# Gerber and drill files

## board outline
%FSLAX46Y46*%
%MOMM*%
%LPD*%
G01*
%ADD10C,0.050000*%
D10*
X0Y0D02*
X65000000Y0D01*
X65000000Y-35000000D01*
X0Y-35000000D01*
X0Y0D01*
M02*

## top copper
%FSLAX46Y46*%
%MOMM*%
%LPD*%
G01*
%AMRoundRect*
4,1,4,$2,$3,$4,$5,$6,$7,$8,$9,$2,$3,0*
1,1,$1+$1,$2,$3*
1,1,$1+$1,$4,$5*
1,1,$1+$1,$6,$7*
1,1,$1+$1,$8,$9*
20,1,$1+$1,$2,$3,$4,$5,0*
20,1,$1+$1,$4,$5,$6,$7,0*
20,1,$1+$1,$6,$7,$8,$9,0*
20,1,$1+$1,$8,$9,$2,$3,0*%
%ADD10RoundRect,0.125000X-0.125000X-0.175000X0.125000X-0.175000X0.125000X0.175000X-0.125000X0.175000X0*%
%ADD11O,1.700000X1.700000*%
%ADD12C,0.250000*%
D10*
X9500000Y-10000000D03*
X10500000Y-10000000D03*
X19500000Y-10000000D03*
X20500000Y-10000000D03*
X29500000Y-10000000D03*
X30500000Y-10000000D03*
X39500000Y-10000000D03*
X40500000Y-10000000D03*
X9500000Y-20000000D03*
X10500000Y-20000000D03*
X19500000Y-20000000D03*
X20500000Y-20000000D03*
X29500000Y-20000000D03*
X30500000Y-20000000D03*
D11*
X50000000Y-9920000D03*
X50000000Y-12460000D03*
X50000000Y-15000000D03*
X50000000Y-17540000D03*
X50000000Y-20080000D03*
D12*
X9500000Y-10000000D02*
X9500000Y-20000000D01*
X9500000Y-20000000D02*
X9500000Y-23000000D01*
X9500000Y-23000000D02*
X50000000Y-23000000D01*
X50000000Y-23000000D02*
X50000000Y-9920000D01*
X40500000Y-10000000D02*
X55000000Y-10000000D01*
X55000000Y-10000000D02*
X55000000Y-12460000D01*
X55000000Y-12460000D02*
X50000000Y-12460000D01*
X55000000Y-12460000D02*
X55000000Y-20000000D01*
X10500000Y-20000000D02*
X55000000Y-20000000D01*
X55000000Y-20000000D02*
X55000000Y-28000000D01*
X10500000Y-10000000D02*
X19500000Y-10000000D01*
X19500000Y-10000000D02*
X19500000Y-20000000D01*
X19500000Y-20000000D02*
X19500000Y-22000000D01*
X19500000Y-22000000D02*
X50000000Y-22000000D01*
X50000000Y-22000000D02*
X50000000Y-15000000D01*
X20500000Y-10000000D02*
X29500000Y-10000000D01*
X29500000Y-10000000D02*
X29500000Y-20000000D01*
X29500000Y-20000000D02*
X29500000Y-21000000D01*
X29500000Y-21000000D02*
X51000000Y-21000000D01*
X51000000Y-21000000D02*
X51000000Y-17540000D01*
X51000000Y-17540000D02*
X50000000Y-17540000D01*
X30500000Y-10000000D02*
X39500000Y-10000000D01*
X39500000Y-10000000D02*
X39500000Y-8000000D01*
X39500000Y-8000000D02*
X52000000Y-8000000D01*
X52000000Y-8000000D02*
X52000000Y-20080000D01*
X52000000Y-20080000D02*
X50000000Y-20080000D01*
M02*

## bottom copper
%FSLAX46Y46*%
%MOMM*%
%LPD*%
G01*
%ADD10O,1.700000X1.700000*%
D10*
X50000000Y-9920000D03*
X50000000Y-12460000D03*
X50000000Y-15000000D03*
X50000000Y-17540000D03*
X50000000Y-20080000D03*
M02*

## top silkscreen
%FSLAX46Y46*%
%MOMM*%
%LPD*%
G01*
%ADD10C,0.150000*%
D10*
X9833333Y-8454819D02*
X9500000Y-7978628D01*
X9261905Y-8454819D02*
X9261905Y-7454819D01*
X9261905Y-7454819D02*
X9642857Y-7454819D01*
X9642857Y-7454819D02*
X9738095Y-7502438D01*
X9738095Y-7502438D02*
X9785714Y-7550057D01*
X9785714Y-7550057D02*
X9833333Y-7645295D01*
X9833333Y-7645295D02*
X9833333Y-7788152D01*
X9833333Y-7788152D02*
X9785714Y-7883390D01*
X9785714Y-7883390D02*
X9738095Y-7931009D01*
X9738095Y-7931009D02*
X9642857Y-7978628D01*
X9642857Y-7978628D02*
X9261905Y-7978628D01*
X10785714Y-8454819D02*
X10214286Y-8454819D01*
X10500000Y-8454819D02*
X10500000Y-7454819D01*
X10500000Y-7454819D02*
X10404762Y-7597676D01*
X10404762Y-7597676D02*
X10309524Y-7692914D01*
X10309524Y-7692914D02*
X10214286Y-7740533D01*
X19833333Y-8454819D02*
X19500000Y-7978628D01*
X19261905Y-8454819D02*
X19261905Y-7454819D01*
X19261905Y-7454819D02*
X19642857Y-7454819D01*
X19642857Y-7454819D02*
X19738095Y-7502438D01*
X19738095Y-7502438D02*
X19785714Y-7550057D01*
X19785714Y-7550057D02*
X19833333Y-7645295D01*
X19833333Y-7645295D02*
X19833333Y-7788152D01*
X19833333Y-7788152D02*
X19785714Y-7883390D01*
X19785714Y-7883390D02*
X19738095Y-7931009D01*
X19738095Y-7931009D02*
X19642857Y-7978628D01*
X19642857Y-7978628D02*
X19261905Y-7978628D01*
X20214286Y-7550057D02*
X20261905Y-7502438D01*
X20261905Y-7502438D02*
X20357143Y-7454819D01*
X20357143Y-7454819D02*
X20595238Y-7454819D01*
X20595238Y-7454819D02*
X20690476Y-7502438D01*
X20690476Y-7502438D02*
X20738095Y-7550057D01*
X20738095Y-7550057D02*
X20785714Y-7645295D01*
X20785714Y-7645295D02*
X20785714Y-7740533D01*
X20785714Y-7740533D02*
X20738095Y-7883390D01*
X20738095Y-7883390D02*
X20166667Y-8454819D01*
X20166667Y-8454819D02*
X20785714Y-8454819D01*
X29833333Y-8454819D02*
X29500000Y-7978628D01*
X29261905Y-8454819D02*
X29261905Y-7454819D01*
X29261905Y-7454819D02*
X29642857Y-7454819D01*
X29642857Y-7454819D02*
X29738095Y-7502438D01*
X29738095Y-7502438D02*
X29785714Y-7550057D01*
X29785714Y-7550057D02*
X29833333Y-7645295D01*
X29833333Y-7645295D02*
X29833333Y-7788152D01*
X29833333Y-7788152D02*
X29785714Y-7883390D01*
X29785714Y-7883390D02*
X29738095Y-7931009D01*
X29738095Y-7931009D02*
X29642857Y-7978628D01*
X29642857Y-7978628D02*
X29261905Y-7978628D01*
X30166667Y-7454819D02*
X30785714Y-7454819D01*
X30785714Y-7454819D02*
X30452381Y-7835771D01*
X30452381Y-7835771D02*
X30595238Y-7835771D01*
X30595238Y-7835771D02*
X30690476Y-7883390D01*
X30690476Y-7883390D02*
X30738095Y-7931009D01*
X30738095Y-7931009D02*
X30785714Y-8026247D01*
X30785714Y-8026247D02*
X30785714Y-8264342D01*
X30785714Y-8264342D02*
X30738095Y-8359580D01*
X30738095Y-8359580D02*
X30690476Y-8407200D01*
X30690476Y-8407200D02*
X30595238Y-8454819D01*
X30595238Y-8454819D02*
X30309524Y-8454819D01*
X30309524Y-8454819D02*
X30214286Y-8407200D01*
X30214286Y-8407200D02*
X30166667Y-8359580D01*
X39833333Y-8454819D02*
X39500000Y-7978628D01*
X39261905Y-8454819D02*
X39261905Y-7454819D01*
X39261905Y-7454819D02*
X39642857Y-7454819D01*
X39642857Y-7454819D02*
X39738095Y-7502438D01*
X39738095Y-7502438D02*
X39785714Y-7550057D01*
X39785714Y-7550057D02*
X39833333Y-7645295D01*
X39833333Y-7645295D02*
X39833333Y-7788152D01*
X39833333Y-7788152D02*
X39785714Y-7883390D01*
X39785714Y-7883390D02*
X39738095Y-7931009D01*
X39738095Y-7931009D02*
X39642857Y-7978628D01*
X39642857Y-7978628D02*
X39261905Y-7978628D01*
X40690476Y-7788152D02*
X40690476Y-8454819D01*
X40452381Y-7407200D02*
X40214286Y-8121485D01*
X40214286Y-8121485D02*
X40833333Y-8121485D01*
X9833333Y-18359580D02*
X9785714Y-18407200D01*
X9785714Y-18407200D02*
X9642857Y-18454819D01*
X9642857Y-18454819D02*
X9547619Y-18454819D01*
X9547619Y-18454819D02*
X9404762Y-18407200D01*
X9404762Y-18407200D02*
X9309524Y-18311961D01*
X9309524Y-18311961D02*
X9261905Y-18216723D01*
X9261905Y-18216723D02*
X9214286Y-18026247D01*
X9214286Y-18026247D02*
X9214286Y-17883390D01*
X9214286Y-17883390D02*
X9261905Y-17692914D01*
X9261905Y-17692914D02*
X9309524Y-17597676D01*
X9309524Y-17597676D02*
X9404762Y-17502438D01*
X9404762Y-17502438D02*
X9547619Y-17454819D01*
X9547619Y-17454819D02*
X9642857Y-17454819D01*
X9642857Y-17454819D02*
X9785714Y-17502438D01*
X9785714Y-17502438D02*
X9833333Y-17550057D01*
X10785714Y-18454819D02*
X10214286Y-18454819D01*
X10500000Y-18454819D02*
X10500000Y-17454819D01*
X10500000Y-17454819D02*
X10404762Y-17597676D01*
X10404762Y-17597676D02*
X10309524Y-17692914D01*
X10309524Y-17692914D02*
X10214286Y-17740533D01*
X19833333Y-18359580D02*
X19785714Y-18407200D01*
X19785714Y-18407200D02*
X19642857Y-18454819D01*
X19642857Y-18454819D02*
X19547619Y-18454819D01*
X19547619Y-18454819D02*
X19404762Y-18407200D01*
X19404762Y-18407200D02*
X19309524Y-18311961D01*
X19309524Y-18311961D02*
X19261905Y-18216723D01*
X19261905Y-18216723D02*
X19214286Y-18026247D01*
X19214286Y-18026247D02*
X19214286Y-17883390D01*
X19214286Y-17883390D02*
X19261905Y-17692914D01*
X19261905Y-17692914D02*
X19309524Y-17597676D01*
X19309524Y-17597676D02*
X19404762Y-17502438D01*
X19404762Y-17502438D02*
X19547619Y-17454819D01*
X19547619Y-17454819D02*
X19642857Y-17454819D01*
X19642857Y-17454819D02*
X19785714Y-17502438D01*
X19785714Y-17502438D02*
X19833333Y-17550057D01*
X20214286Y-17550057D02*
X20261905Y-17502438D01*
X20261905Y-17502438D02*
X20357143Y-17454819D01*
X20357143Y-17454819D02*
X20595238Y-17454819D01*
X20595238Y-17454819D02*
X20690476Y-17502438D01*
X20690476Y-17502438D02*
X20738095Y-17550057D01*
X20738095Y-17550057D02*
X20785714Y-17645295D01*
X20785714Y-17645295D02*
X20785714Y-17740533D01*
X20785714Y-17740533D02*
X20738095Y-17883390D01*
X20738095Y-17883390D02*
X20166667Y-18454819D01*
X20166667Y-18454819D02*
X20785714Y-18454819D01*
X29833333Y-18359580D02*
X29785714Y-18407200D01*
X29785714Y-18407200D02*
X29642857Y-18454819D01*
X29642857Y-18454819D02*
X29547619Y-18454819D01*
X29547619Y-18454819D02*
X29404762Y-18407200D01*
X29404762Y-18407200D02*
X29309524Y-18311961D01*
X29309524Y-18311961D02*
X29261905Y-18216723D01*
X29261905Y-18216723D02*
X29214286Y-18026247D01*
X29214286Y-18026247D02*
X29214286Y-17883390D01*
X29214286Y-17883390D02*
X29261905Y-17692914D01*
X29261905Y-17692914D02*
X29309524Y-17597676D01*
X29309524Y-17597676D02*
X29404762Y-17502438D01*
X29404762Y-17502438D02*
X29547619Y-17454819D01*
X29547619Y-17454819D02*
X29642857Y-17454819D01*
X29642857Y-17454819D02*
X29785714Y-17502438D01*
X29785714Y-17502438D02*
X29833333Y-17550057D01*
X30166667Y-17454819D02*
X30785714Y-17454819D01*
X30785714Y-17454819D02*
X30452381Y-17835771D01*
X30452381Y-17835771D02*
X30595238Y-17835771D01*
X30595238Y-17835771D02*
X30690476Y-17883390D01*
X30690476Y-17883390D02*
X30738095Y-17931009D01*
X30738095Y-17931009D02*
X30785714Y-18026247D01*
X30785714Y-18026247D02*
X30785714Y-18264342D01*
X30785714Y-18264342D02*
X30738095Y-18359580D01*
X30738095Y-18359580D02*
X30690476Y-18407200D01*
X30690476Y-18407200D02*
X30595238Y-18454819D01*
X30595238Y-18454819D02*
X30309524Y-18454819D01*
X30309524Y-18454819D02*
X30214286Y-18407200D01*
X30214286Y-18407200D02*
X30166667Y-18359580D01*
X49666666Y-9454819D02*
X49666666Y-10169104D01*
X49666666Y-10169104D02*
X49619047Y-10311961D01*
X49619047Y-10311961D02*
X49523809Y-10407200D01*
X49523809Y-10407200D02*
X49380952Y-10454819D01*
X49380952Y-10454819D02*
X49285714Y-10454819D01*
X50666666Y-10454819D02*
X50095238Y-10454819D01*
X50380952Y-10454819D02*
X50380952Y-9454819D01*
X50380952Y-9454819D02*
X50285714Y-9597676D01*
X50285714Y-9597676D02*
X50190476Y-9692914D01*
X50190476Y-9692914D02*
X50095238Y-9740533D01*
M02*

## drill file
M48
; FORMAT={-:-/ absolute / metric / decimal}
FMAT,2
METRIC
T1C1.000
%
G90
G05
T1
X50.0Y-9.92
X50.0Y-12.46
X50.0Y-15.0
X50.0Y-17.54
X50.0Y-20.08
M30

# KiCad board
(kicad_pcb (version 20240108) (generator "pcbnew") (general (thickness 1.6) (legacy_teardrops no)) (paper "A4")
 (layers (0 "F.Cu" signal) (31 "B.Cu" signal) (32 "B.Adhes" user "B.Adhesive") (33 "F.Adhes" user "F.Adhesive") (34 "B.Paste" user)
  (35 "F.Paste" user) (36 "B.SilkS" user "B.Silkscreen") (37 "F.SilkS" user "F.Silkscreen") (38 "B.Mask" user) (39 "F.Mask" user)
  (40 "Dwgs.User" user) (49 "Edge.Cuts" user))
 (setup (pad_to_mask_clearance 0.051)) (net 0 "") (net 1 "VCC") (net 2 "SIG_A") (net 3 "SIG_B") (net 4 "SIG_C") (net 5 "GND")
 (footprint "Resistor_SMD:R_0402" (layer "F.Cu") (at 10 10)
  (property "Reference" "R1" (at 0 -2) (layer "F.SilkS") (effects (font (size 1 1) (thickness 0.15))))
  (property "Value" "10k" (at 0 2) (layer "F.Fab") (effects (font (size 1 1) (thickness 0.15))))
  (pad "1" smd roundrect (at -0.5 0) (size 0.5 0.6) (layers "F.Cu" "F.Paste" "F.Mask") (roundrect_rratio 0.25) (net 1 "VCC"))
  (pad "2" smd roundrect (at 0.5 0) (size 0.5 0.6) (layers "F.Cu" "F.Paste" "F.Mask") (roundrect_rratio 0.25) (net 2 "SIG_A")))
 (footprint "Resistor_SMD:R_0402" (layer "F.Cu") (at 20 10)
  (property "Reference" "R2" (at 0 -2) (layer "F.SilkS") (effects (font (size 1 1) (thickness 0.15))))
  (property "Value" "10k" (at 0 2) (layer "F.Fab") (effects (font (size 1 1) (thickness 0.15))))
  (pad "1" smd roundrect (at -0.5 0) (size 0.5 0.6) (layers "F.Cu" "F.Paste" "F.Mask") (roundrect_rratio 0.25) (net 2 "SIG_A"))
  (pad "2" smd roundrect (at 0.5 0) (size 0.5 0.6) (layers "F.Cu" "F.Paste" "F.Mask") (roundrect_rratio 0.25) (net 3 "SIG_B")))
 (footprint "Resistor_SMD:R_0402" (layer "F.Cu") (at 30 10)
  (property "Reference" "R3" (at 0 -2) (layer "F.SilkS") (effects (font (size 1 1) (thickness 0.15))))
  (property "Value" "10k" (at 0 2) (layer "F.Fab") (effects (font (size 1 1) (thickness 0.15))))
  (pad "1" smd roundrect (at -0.5 0) (size 0.5 0.6) (layers "F.Cu" "F.Paste" "F.Mask") (roundrect_rratio 0.25) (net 3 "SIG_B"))
  (pad "2" smd roundrect (at 0.5 0) (size 0.5 0.6) (layers "F.Cu" "F.Paste" "F.Mask") (roundrect_rratio 0.25) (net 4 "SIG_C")))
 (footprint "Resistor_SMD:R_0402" (layer "F.Cu") (at 40 10)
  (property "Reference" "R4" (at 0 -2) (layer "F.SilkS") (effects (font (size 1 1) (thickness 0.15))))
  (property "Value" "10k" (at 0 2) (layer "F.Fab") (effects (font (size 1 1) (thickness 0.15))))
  (pad "1" smd roundrect (at -0.5 0) (size 0.5 0.6) (layers "F.Cu" "F.Paste" "F.Mask") (roundrect_rratio 0.25) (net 4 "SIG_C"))
  (pad "2" smd roundrect (at 0.5 0) (size 0.5 0.6) (layers "F.Cu" "F.Paste" "F.Mask") (roundrect_rratio 0.25) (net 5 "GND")))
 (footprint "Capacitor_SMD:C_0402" (layer "F.Cu") (at 10 20)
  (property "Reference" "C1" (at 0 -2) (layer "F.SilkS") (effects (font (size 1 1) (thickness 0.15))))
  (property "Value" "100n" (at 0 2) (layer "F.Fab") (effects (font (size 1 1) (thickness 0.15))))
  (pad "1" smd roundrect (at -0.5 0) (size 0.5 0.6) (layers "F.Cu" "F.Paste" "F.Mask") (roundrect_rratio 0.25) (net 1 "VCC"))
  (pad "2" smd roundrect (at 0.5 0) (size 0.5 0.6) (layers "F.Cu" "F.Paste" "F.Mask") (roundrect_rratio 0.25) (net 5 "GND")))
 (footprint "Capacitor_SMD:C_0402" (layer "F.Cu") (at 20 20)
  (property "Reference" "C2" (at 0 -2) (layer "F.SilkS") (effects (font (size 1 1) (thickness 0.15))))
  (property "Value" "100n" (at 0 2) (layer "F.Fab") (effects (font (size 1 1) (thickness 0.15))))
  (pad "1" smd roundrect (at -0.5 0) (size 0.5 0.6) (layers "F.Cu" "F.Paste" "F.Mask") (roundrect_rratio 0.25) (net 2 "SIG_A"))
  (pad "2" smd roundrect (at 0.5 0) (size 0.5 0.6) (layers "F.Cu" "F.Paste" "F.Mask") (roundrect_rratio 0.25) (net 5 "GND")))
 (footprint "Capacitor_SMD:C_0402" (layer "F.Cu") (at 30 20)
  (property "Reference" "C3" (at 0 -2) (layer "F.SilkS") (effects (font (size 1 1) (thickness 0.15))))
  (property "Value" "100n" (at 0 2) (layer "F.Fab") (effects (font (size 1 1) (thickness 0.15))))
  (pad "1" smd roundrect (at -0.5 0) (size 0.5 0.6) (layers "F.Cu" "F.Paste" "F.Mask") (roundrect_rratio 0.25) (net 3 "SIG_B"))
  (pad "2" smd roundrect (at 0.5 0) (size 0.5 0.6) (layers "F.Cu" "F.Paste" "F.Mask") (roundrect_rratio 0.25) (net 5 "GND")))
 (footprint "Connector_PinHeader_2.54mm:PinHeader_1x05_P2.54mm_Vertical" (layer "F.Cu") (at 50 15)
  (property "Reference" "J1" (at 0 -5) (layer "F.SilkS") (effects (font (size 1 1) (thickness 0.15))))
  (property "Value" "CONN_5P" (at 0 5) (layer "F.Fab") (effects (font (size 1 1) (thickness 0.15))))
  (pad "1" thru_hole oval (at 0 -5.08) (size 1.7 1.7) (drill 1.0) (layers "*.Cu" "*.Mask") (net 1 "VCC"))
  (pad "2" thru_hole oval (at 0 -2.54) (size 1.7 1.7) (drill 1.0) (layers "*.Cu" "*.Mask") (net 5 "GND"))
  (pad "3" thru_hole oval (at 0 0) (size 1.7 1.7) (drill 1.0) (layers "*.Cu" "*.Mask") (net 2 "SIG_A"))
  (pad "4" thru_hole oval (at 0 2.54) (size 1.7 1.7) (drill 1.0) (layers "*.Cu" "*.Mask") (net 3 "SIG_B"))
  (pad "5" thru_hole oval (at 0 5.08) (size 1.7 1.7) (drill 1.0) (layers "*.Cu" "*.Mask") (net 4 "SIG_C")))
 (gr_rect (start 0 0) (end 65 35) (layer "Edge.Cuts") (width 0.05))
 (segment (start 9.5 10) (end 9.5 20) (width 0.25) (layer "F.Cu") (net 1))
 (segment (start 9.5 20) (end 9.5 23) (width 0.25) (layer "F.Cu") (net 1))
 (segment (start 9.5 23) (end 50 23) (width 0.25) (layer "F.Cu") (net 1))
 (segment (start 50 23) (end 50 9.92) (width 0.25) (layer "F.Cu") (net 1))
 (segment (start 40.5 10) (end 55 10) (width 0.25) (layer "F.Cu") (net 5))
 (segment (start 55 10) (end 55 12.46) (width 0.25) (layer "F.Cu") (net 5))
 (segment (start 55 12.46) (end 50 12.46) (width 0.25) (layer "F.Cu") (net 5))
 (segment (start 55 12.46) (end 55 20) (width 0.25) (layer "F.Cu") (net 5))
 (segment (start 10.5 20) (end 55 20) (width 0.25) (layer "F.Cu") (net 5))
 (segment (start 55 20) (end 55 28) (width 0.25) (layer "F.Cu") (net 5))
 (segment (start 10.5 10) (end 19.5 10) (width 0.25) (layer "F.Cu") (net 2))
 (segment (start 19.5 10) (end 19.5 20) (width 0.25) (layer "F.Cu") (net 2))
 (segment (start 19.5 20) (end 19.5 22) (width 0.25) (layer "F.Cu") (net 2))
 (segment (start 19.5 22) (end 50 22) (width 0.25) (layer "F.Cu") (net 2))
 (segment (start 50 22) (end 50 15) (width 0.25) (layer "F.Cu") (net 2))
 (segment (start 20.5 10) (end 29.5 10) (width 0.25) (layer "F.Cu") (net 3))
 (segment (start 29.5 10) (end 29.5 20) (width 0.25) (layer "F.Cu") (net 3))
 (segment (start 29.5 20) (end 29.5 21) (width 0.25) (layer "F.Cu") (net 3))
 (segment (start 29.5 21) (end 51 21) (width 0.25) (layer "F.Cu") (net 3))
 (segment (start 51 21) (end 51 17.54) (width 0.25) (layer "F.Cu") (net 3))
 (segment (start 51 17.54) (end 50 17.54) (width 0.25) (layer "F.Cu") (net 3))
 (segment (start 30.5 10) (end 39.5 10) (width 0.25) (layer "F.Cu") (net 4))
 (segment (start 39.5 10) (end 39.5 8) (width 0.25) (layer "F.Cu") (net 4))
 (segment (start 39.5 8) (end 52 8) (width 0.25) (layer "F.Cu") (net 4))
 (segment (start 52 8) (end 52 20.08) (width 0.25) (layer "F.Cu") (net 4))
 (segment (start 52 20.08) (end 50 20.08) (width 0.25) (layer "F.Cu") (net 4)))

